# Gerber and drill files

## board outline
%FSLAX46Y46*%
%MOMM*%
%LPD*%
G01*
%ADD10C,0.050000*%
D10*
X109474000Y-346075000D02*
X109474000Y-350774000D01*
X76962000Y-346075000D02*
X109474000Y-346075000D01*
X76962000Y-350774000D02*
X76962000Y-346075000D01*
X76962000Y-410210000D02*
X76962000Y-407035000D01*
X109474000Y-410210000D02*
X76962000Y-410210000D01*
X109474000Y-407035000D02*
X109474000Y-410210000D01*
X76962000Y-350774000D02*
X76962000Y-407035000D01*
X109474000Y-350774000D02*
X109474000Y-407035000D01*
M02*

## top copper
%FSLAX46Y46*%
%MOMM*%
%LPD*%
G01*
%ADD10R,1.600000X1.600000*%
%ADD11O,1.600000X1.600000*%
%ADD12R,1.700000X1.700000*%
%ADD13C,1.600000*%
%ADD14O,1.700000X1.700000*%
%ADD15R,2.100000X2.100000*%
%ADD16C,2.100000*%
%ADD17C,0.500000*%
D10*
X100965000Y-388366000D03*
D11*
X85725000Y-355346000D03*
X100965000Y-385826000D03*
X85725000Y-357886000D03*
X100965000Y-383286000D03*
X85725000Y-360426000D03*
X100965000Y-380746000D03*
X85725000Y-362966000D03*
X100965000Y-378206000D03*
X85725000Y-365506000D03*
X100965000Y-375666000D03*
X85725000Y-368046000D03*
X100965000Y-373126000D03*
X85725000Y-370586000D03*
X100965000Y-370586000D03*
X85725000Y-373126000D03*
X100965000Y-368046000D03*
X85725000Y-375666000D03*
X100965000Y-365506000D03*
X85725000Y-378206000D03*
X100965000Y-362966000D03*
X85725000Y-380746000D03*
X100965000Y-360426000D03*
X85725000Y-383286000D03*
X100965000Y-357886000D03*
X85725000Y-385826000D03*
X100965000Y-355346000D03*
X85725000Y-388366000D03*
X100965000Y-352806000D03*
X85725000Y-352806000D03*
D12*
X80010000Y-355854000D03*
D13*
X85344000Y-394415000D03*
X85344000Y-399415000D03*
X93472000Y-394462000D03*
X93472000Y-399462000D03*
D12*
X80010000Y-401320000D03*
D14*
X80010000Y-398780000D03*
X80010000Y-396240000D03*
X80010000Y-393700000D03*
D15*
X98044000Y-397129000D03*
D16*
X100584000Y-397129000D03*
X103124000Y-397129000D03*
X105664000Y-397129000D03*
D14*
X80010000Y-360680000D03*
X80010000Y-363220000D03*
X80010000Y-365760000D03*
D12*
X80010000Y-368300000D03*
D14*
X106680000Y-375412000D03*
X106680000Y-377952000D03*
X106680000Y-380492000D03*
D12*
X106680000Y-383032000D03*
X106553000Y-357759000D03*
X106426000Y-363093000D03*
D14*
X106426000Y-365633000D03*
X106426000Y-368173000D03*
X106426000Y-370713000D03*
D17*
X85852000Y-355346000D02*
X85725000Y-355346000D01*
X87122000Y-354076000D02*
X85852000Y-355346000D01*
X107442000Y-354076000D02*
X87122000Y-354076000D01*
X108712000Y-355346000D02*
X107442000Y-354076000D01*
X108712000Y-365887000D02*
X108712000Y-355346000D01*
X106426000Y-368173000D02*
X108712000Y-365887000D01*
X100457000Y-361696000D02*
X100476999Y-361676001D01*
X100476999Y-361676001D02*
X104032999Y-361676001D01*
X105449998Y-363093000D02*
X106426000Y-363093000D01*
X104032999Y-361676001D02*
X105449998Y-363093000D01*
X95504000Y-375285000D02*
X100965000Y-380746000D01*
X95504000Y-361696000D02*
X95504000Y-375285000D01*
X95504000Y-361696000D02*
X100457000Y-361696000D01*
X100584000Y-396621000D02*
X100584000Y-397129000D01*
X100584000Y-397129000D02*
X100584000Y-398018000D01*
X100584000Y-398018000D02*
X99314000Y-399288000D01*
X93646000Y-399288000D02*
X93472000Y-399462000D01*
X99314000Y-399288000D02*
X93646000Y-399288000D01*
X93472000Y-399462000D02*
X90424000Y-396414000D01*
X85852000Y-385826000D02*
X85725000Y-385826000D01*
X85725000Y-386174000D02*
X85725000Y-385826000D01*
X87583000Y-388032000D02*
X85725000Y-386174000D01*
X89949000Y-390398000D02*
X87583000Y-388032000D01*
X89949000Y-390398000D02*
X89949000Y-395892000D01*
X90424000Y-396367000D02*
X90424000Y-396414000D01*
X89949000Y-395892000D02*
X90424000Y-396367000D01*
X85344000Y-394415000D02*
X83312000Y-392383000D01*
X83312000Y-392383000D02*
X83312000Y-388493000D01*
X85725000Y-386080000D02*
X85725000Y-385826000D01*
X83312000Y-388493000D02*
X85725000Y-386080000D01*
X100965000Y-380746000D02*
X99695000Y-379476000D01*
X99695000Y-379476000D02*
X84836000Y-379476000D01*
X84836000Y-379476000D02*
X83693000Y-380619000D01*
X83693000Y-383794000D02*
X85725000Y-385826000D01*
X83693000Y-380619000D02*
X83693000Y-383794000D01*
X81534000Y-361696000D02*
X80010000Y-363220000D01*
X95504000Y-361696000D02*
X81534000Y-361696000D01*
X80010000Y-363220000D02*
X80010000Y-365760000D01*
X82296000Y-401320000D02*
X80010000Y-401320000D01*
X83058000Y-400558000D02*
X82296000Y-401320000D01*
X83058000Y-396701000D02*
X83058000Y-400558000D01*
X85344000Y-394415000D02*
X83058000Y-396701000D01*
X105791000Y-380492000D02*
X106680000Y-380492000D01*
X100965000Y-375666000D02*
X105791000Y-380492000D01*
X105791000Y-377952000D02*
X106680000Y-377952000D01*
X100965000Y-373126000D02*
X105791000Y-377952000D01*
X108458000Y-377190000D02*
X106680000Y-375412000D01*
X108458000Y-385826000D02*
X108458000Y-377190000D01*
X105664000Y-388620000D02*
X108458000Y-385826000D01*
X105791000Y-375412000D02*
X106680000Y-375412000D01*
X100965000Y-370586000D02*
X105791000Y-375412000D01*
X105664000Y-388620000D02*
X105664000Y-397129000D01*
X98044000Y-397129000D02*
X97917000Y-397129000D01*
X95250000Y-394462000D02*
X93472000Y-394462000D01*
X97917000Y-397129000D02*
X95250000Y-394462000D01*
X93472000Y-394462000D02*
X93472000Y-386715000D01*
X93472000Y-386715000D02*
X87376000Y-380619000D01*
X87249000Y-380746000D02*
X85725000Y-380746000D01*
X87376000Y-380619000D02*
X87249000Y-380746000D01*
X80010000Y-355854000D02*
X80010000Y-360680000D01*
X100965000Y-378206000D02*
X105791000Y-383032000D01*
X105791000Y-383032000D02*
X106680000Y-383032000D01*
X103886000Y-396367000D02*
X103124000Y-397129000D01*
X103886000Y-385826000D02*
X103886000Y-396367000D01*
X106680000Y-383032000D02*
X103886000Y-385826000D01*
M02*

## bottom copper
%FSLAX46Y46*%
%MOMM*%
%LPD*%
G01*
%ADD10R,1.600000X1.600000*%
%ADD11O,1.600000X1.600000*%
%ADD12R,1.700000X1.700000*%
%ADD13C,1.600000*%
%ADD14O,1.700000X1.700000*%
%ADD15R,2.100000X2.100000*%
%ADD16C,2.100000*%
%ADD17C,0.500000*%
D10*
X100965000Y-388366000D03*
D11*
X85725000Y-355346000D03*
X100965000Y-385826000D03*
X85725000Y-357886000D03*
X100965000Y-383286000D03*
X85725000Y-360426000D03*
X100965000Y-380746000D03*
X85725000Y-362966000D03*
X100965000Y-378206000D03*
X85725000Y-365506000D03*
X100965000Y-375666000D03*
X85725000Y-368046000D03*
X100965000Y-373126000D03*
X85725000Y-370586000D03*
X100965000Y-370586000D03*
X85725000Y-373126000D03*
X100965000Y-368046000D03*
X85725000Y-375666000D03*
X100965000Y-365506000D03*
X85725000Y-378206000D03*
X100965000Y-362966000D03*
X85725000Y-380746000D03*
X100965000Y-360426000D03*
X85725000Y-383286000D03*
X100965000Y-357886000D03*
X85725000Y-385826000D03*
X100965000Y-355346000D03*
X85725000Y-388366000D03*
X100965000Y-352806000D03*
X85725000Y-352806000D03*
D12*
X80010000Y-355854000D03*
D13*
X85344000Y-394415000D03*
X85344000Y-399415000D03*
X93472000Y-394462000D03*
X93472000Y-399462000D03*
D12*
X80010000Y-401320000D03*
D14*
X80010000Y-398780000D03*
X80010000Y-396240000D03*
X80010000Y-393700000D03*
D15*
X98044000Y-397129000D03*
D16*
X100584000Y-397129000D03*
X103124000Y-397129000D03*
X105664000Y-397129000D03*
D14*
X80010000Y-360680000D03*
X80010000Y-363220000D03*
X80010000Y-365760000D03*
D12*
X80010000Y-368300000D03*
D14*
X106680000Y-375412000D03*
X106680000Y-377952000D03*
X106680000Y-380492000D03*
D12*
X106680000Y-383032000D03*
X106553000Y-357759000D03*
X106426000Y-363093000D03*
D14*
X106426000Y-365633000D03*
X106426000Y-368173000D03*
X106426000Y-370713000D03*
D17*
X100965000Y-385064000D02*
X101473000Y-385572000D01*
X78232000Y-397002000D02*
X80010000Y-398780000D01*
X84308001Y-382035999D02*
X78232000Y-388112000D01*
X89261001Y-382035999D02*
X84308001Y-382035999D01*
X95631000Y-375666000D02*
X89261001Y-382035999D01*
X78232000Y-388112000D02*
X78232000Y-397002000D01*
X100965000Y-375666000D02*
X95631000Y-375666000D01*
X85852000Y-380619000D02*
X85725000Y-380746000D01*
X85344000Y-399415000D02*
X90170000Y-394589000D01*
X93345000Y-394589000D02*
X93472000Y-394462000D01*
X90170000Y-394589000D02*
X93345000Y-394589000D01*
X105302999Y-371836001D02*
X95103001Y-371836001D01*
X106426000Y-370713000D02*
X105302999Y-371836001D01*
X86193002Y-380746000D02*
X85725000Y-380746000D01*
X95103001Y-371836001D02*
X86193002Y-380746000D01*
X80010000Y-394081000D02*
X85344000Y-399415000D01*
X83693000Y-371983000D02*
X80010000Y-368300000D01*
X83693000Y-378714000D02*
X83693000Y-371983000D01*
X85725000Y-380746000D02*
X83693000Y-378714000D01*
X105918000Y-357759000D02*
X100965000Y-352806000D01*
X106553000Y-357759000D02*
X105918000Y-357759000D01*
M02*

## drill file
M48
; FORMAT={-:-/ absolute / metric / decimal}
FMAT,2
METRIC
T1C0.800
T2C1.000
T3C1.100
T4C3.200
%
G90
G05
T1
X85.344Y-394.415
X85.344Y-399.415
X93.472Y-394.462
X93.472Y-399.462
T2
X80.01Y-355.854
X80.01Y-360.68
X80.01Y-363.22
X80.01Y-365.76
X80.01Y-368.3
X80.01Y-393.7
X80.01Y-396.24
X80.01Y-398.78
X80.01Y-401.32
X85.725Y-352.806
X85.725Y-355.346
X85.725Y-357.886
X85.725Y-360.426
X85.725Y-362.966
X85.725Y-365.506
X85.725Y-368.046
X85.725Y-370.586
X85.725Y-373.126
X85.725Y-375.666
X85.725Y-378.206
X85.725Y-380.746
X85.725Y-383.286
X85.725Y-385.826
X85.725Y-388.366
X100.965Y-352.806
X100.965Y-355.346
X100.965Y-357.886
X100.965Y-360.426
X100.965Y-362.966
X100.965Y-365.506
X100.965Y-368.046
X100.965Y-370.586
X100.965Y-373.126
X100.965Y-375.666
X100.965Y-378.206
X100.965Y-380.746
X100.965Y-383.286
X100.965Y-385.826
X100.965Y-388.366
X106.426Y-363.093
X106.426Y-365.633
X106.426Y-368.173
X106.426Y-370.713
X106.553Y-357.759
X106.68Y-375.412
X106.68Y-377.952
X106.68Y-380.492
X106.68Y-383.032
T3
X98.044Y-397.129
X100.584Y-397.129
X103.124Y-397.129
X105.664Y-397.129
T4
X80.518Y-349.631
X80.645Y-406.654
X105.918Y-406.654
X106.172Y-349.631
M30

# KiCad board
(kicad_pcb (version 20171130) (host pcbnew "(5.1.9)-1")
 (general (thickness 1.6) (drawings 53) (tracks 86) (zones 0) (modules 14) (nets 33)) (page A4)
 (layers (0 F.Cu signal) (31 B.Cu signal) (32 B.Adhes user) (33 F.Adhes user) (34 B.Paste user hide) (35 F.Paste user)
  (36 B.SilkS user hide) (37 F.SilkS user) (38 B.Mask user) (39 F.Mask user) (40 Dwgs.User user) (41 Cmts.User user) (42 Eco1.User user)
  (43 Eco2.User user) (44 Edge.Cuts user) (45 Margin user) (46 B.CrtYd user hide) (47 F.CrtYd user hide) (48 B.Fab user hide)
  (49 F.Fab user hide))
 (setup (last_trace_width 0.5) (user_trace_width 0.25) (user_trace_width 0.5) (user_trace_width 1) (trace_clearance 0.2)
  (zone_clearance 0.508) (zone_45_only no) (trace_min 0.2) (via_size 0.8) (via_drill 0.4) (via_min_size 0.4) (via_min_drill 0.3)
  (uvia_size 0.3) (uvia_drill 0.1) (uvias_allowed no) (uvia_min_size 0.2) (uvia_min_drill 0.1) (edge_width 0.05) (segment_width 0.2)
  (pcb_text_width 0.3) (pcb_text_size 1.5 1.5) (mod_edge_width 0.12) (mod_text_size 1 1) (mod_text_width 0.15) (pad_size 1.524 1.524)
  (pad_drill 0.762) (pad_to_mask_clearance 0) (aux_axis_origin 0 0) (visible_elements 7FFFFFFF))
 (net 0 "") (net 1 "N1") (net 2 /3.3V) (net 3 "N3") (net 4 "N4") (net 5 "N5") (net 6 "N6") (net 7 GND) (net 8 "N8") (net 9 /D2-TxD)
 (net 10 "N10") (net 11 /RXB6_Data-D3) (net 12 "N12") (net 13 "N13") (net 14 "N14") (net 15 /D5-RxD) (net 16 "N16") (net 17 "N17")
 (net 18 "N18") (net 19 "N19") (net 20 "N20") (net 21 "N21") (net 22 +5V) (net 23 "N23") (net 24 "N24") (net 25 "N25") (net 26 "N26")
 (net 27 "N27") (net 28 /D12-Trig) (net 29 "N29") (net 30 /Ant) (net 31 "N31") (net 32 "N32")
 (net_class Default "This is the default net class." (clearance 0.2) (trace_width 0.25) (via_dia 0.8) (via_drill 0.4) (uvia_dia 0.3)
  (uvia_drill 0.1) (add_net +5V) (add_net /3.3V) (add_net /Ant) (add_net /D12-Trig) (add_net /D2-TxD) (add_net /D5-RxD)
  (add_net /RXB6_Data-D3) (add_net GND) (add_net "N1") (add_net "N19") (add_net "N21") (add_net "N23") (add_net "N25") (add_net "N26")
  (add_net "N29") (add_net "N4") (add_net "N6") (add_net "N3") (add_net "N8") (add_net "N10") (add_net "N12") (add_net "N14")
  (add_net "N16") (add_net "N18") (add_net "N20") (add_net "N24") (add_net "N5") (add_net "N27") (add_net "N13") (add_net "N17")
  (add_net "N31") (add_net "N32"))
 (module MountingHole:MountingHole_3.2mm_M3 (layer F.Cu) (at 106.172 349.631)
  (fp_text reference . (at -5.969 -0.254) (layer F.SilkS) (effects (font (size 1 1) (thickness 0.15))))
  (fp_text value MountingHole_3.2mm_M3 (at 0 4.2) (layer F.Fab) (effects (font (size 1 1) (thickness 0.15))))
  (pad 1 np_thru_hole circle (at 0 0) (size 3.2 3.2) (drill 3.2) (layers *.Cu *.Mask)))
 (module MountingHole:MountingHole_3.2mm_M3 (layer F.Cu) (at 80.518 349.631)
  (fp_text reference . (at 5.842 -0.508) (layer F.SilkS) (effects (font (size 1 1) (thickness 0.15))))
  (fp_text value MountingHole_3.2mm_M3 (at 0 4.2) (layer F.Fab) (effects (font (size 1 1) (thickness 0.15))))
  (pad 1 np_thru_hole circle (at 0 0) (size 3.2 3.2) (drill 3.2) (layers *.Cu *.Mask)))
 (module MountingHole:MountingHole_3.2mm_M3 (layer F.Cu) (at 105.918 406.654)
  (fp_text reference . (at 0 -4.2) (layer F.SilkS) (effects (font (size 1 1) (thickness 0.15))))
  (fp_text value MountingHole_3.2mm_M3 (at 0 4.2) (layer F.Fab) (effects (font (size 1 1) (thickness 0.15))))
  (pad 1 np_thru_hole circle (at 0 0) (size 3.2 3.2) (drill 3.2) (layers *.Cu *.Mask)))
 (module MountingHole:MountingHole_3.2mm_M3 (layer F.Cu) (at 80.645 406.654)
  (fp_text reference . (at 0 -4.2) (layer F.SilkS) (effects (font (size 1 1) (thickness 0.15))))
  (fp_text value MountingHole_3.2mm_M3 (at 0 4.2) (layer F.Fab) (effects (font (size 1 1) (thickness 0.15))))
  (pad 1 np_thru_hole circle (at 0 0) (size 3.2 3.2) (drill 3.2) (layers *.Cu *.Mask)))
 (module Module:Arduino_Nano (layer F.Cu) (at 100.965 388.366 180)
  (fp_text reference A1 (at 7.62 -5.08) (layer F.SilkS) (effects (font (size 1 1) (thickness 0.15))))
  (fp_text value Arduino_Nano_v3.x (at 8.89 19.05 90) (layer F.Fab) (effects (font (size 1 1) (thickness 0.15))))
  (pad 1 thru_hole rect (at 0 0 180) (size 1.6 1.6) (drill 1) (layers *.Cu *.Mask) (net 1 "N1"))
  (pad 17 thru_hole oval (at 15.24 33.02 180) (size 1.6 1.6) (drill 1) (layers *.Cu *.Mask) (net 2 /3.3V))
  (pad 2 thru_hole oval (at 0 2.54 180) (size 1.6 1.6) (drill 1) (layers *.Cu *.Mask) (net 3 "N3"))
  (pad 18 thru_hole oval (at 15.24 30.48 180) (size 1.6 1.6) (drill 1) (layers *.Cu *.Mask) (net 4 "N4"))
  (pad 3 thru_hole oval (at 0 5.08 180) (size 1.6 1.6) (drill 1) (layers *.Cu *.Mask) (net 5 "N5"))
  (pad 19 thru_hole oval (at 15.24 27.94 180) (size 1.6 1.6) (drill 1) (layers *.Cu *.Mask) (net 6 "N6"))
  (pad 4 thru_hole oval (at 0 7.62 180) (size 1.6 1.6) (drill 1) (layers *.Cu *.Mask) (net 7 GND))
  (pad 20 thru_hole oval (at 15.24 25.4 180) (size 1.6 1.6) (drill 1) (layers *.Cu *.Mask) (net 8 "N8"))
  (pad 5 thru_hole oval (at 0 10.16 180) (size 1.6 1.6) (drill 1) (layers *.Cu *.Mask) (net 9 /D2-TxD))
  (pad 21 thru_hole oval (at 15.24 22.86 180) (size 1.6 1.6) (drill 1) (layers *.Cu *.Mask) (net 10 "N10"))
  (pad 6 thru_hole oval (at 0 12.7 180) (size 1.6 1.6) (drill 1) (layers *.Cu *.Mask) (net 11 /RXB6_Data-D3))
  (pad 22 thru_hole oval (at 15.24 20.32 180) (size 1.6 1.6) (drill 1) (layers *.Cu *.Mask) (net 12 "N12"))
  (pad 7 thru_hole oval (at 0 15.24 180) (size 1.6 1.6) (drill 1) (layers *.Cu *.Mask) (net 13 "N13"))
  (pad 23 thru_hole oval (at 15.24 17.78 180) (size 1.6 1.6) (drill 1) (layers *.Cu *.Mask) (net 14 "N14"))
  (pad 8 thru_hole oval (at 0 17.78 180) (size 1.6 1.6) (drill 1) (layers *.Cu *.Mask) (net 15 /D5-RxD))
  (pad 24 thru_hole oval (at 15.24 15.24 180) (size 1.6 1.6) (drill 1) (layers *.Cu *.Mask) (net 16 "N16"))
  (pad 9 thru_hole oval (at 0 20.32 180) (size 1.6 1.6) (drill 1) (layers *.Cu *.Mask) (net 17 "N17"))
  (pad 25 thru_hole oval (at 15.24 12.7 180) (size 1.6 1.6) (drill 1) (layers *.Cu *.Mask) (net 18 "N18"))
  (pad 10 thru_hole oval (at 0 22.86 180) (size 1.6 1.6) (drill 1) (layers *.Cu *.Mask) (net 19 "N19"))
  (pad 26 thru_hole oval (at 15.24 10.16 180) (size 1.6 1.6) (drill 1) (layers *.Cu *.Mask) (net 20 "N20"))
  (pad 11 thru_hole oval (at 0 25.4 180) (size 1.6 1.6) (drill 1) (layers *.Cu *.Mask) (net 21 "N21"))
  (pad 27 thru_hole oval (at 15.24 7.62 180) (size 1.6 1.6) (drill 1) (layers *.Cu *.Mask) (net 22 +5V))
  (pad 12 thru_hole oval (at 0 27.94 180) (size 1.6 1.6) (drill 1) (layers *.Cu *.Mask) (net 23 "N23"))
  (pad 28 thru_hole oval (at 15.24 5.08 180) (size 1.6 1.6) (drill 1) (layers *.Cu *.Mask) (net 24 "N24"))
  (pad 13 thru_hole oval (at 0 30.48 180) (size 1.6 1.6) (drill 1) (layers *.Cu *.Mask) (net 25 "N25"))
  (pad 29 thru_hole oval (at 15.24 2.54 180) (size 1.6 1.6) (drill 1) (layers *.Cu *.Mask) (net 7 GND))
  (pad 14 thru_hole oval (at 0 33.02 180) (size 1.6 1.6) (drill 1) (layers *.Cu *.Mask) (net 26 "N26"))
  (pad 30 thru_hole oval (at 15.24 0 180) (size 1.6 1.6) (drill 1) (layers *.Cu *.Mask) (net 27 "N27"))
  (pad 15 thru_hole oval (at 0 35.56 180) (size 1.6 1.6) (drill 1) (layers *.Cu *.Mask) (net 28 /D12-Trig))
  (pad 16 thru_hole oval (at 15.24 35.56 180) (size 1.6 1.6) (drill 1) (layers *.Cu *.Mask) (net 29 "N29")))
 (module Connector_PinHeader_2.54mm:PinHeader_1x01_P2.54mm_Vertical (layer F.Cu) (at 80.01 355.854)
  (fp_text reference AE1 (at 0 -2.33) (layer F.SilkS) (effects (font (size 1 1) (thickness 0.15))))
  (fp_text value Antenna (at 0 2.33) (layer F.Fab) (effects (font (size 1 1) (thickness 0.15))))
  (pad 1 thru_hole rect (at 0 0) (size 1.7 1.7) (drill 1) (layers *.Cu *.Mask) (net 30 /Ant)))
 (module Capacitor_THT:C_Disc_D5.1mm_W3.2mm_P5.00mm (layer F.Cu) (at 85.344 399.415 90)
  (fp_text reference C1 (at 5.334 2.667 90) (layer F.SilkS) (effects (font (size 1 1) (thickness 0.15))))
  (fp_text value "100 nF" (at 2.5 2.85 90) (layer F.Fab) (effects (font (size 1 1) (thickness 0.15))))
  (pad 2 thru_hole circle (at 5 0 90) (size 1.6 1.6) (drill 0.8) (layers *.Cu *.Mask) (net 7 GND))
  (pad 1 thru_hole circle (at 0 0 90) (size 1.6 1.6) (drill 0.8) (layers *.Cu *.Mask) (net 22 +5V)))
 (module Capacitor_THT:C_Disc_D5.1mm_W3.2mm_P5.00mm (layer F.Cu) (at 93.472 394.462 270)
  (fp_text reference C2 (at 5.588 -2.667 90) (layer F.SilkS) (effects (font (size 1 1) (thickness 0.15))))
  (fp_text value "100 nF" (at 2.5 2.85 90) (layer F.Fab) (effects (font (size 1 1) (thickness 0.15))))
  (pad 1 thru_hole circle (at 0 0 270) (size 1.6 1.6) (drill 0.8) (layers *.Cu *.Mask) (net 22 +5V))
  (pad 2 thru_hole circle (at 5 0 270) (size 1.6 1.6) (drill 0.8) (layers *.Cu *.Mask) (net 7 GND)))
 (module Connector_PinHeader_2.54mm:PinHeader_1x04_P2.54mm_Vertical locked (layer F.Cu) (at 80.01 401.32 180)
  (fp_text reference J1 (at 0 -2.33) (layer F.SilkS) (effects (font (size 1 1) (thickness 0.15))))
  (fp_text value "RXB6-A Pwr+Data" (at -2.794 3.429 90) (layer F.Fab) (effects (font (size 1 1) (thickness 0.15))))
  (pad 1 thru_hole rect (at 0 0 180) (size 1.7 1.7) (drill 1) (layers *.Cu *.Mask) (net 7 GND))
  (pad 2 thru_hole oval (at 0 2.54 180) (size 1.7 1.7) (drill 1) (layers *.Cu *.Mask) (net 11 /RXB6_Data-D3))
  (pad 3 thru_hole oval (at 0 5.08 180) (size 1.7 1.7) (drill 1) (layers *.Cu *.Mask) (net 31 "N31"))
  (pad 4 thru_hole oval (at 0 7.62 180) (size 1.7 1.7) (drill 1) (layers *.Cu *.Mask) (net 22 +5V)))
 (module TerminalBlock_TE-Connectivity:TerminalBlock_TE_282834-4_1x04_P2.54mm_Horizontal (layer F.Cu) (at 98.044 397.129)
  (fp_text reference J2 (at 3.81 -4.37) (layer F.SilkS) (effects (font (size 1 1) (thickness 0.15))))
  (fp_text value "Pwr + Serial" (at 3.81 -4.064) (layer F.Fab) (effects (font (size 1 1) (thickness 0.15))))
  (pad 1 thru_hole rect (at 0 0) (size 2.1 2.1) (drill 1.1) (layers *.Cu *.Mask) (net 22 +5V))
  (pad 2 thru_hole circle (at 2.54 0) (size 2.1 2.1) (drill 1.1) (layers *.Cu *.Mask) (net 7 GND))
  (pad 3 thru_hole circle (at 5.08 0) (size 2.1 2.1) (drill 1.1) (layers *.Cu *.Mask) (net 9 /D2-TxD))
  (pad 4 thru_hole circle (at 7.62 0) (size 2.1 2.1) (drill 1.1) (layers *.Cu *.Mask) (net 15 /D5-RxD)))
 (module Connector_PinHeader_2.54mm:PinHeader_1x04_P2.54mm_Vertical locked (layer F.Cu) (at 80.01 368.3 180)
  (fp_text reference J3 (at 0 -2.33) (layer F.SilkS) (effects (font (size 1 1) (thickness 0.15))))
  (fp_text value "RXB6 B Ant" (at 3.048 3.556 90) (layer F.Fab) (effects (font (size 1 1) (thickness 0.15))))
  (pad 4 thru_hole oval (at 0 7.62 180) (size 1.7 1.7) (drill 1) (layers *.Cu *.Mask) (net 30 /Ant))
  (pad 3 thru_hole oval (at 0 5.08 180) (size 1.7 1.7) (drill 1) (layers *.Cu *.Mask) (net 7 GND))
  (pad 2 thru_hole oval (at 0 2.54 180) (size 1.7 1.7) (drill 1) (layers *.Cu *.Mask) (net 7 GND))
  (pad 1 thru_hole rect (at 0 0 180) (size 1.7 1.7) (drill 1) (layers *.Cu *.Mask) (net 22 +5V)))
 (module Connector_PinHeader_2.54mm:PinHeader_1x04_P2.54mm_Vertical (layer F.Cu) (at 106.68 383.032 180)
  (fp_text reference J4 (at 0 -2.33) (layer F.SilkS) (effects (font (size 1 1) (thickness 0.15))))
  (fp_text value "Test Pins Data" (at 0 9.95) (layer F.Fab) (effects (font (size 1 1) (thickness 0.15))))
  (pad 4 thru_hole oval (at 0 7.62 180) (size 1.7 1.7) (drill 1) (layers *.Cu *.Mask) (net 15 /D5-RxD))
  (pad 3 thru_hole oval (at 0 5.08 180) (size 1.7 1.7) (drill 1) (layers *.Cu *.Mask) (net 13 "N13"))
  (pad 2 thru_hole oval (at 0 2.54 180) (size 1.7 1.7) (drill 1) (layers *.Cu *.Mask) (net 11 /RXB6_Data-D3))
  (pad 1 thru_hole rect (at 0 0 180) (size 1.7 1.7) (drill 1) (layers *.Cu *.Mask) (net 9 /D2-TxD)))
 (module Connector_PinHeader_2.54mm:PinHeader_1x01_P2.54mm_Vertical (layer F.Cu) (at 106.553 357.759)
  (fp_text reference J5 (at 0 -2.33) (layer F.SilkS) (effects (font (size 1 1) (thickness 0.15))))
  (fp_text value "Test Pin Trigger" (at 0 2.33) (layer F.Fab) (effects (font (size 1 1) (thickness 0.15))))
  (pad 1 thru_hole rect (at 0 0) (size 1.7 1.7) (drill 1) (layers *.Cu *.Mask) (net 28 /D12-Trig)))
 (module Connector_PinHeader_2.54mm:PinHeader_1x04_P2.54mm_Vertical (layer F.Cu) (at 106.426 363.093)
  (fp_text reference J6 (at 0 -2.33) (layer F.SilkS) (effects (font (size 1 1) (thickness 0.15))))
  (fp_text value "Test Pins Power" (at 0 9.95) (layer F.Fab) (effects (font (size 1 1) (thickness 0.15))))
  (pad 1 thru_hole rect (at 0 0) (size 1.7 1.7) (drill 1) (layers *.Cu *.Mask) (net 7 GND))
  (pad 2 thru_hole oval (at 0 2.54) (size 1.7 1.7) (drill 1) (layers *.Cu *.Mask) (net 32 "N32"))
  (pad 3 thru_hole oval (at 0 5.08) (size 1.7 1.7) (drill 1) (layers *.Cu *.Mask) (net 2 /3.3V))
  (pad 4 thru_hole oval (at 0 7.62) (size 1.7 1.7) (drill 1) (layers *.Cu *.Mask) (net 22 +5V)))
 (gr_line (start 109.474 346.075) (end 109.474 350.774) (layer Edge.Cuts) (width 0.05))
 (gr_line (start 76.962 346.075) (end 109.474 346.075) (layer Edge.Cuts) (width 0.05))
 (gr_line (start 76.962 350.774) (end 76.962 346.075) (layer Edge.Cuts) (width 0.05))
 (gr_line (start 76.962 410.21) (end 76.962 407.035) (layer Edge.Cuts) (width 0.05))
 (gr_line (start 109.474 410.21) (end 76.962 410.21) (layer Edge.Cuts) (width 0.05))
 (gr_line (start 109.474 407.035) (end 109.474 410.21) (layer Edge.Cuts) (width 0.05))
 (gr_line (start 76.962 350.774) (end 76.962 407.035) (layer Edge.Cuts) (width 0.05))
 (gr_line (start 109.474 350.774) (end 109.474 407.035) (layer Edge.Cuts) (width 0.05))
 (segment (start 85.852 355.346) (end 85.725 355.346) (width 0.5) (layer F.Cu) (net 2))
 (segment (start 87.122 354.076) (end 85.852 355.346) (width 0.5) (layer F.Cu) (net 2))
 (segment (start 107.442 354.076) (end 87.122 354.076) (width 0.5) (layer F.Cu) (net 2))
 (segment (start 108.712 355.346) (end 107.442 354.076) (width 0.5) (layer F.Cu) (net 2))
 (segment (start 108.712 365.887) (end 108.712 355.346) (width 0.5) (layer F.Cu) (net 2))
 (segment (start 106.426 368.173) (end 108.712 365.887) (width 0.5) (layer F.Cu) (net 2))
 (segment (start 100.965 385.064) (end 101.473 385.572) (width 0.5) (layer B.Cu) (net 3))
 (segment (start 100.457 361.696) (end 100.476999 361.676001) (width 0.5) (layer F.Cu) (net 7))
 (segment (start 100.476999 361.676001) (end 104.032999 361.676001) (width 0.5) (layer F.Cu) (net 7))
 (segment (start 105.449998 363.093) (end 106.426 363.093) (width 0.5) (layer F.Cu) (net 7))
 (segment (start 104.032999 361.676001) (end 105.449998 363.093) (width 0.5) (layer F.Cu) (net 7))
 (segment (start 95.504 375.285) (end 100.965 380.746) (width 0.5) (layer F.Cu) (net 7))
 (segment (start 95.504 361.696) (end 95.504 375.285) (width 0.5) (layer F.Cu) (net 7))
 (segment (start 95.504 361.696) (end 100.457 361.696) (width 0.5) (layer F.Cu) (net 7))
 (segment (start 100.584 396.621) (end 100.584 397.129) (width 0.5) (layer F.Cu) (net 7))
 (segment (start 100.584 397.129) (end 100.584 398.018) (width 0.5) (layer F.Cu) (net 7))
 (segment (start 100.584 398.018) (end 99.314 399.288) (width 0.5) (layer F.Cu) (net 7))
 (segment (start 93.646 399.288) (end 93.472 399.462) (width 0.5) (layer F.Cu) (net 7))
 (segment (start 99.314 399.288) (end 93.646 399.288) (width 0.5) (layer F.Cu) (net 7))
 (segment (start 93.472 399.462) (end 90.424 396.414) (width 0.5) (layer F.Cu) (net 7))
 (segment (start 85.852 385.826) (end 85.725 385.826) (width 0.5) (layer F.Cu) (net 7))
 (segment (start 85.725 386.174) (end 85.725 385.826) (width 0.5) (layer F.Cu) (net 7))
 (segment (start 87.583 388.032) (end 85.725 386.174) (width 0.5) (layer F.Cu) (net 7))
 (segment (start 89.949 390.398) (end 87.583 388.032) (width 0.5) (layer F.Cu) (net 7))
 (segment (start 89.949 390.398) (end 89.949 395.892) (width 0.5) (layer F.Cu) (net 7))
 (segment (start 90.424 396.367) (end 90.424 396.414) (width 0.5) (layer F.Cu) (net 7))
 (segment (start 89.949 395.892) (end 90.424 396.367) (width 0.5) (layer F.Cu) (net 7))
 (segment (start 85.344 394.415) (end 83.312 392.383) (width 0.5) (layer F.Cu) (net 7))
 (segment (start 83.312 392.383) (end 83.312 388.493) (width 0.5) (layer F.Cu) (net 7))
 (segment (start 85.725 386.08) (end 85.725 385.826) (width 0.5) (layer F.Cu) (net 7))
 (segment (start 83.312 388.493) (end 85.725 386.08) (width 0.5) (layer F.Cu) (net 7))
 (segment (start 100.965 380.746) (end 99.695 379.476) (width 0.5) (layer F.Cu) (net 7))
 (segment (start 99.695 379.476) (end 84.836 379.476) (width 0.5) (layer F.Cu) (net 7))
 (segment (start 84.836 379.476) (end 83.693 380.619) (width 0.5) (layer F.Cu) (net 7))
 (segment (start 83.693 383.794) (end 85.725 385.826) (width 0.5) (layer F.Cu) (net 7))
 (segment (start 83.693 380.619) (end 83.693 383.794) (width 0.5) (layer F.Cu) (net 7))
 (segment (start 81.534 361.696) (end 80.01 363.22) (width 0.5) (layer F.Cu) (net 7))
 (segment (start 95.504 361.696) (end 81.534 361.696) (width 0.5) (layer F.Cu) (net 7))
 (segment (start 80.01 363.22) (end 80.01 365.76) (width 0.5) (layer F.Cu) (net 7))
 (segment (start 82.296 401.32) (end 80.01 401.32) (width 0.5) (layer F.Cu) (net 7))
 (segment (start 83.058 400.558) (end 82.296 401.32) (width 0.5) (layer F.Cu) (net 7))
 (segment (start 83.058 396.701) (end 83.058 400.558) (width 0.5) (layer F.Cu) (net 7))
 (segment (start 85.344 394.415) (end 83.058 396.701) (width 0.5) (layer F.Cu) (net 7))
 (segment (start 105.791 380.492) (end 106.68 380.492) (width 0.5) (layer F.Cu) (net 11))
 (segment (start 100.965 375.666) (end 105.791 380.492) (width 0.5) (layer F.Cu) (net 11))
 (segment (start 78.232 397.002) (end 80.01 398.78) (width 0.5) (layer B.Cu) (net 11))
 (segment (start 84.308001 382.035999) (end 78.232 388.112) (width 0.5) (layer B.Cu) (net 11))
 (segment (start 89.261001 382.035999) (end 84.308001 382.035999) (width 0.5) (layer B.Cu) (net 11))
 (segment (start 95.631 375.666) (end 89.261001 382.035999) (width 0.5) (layer B.Cu) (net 11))
 (segment (start 78.232 388.112) (end 78.232 397.002) (width 0.5) (layer B.Cu) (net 11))
 (segment (start 100.965 375.666) (end 95.631 375.666) (width 0.5) (layer B.Cu) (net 11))
 (segment (start 105.791 377.952) (end 106.68 377.952) (width 0.5) (layer F.Cu) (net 13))
 (segment (start 100.965 373.126) (end 105.791 377.952) (width 0.5) (layer F.Cu) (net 13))
 (segment (start 108.458 377.19) (end 106.68 375.412) (width 0.5) (layer F.Cu) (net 15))
 (segment (start 108.458 385.826) (end 108.458 377.19) (width 0.5) (layer F.Cu) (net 15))
 (segment (start 105.664 388.62) (end 108.458 385.826) (width 0.5) (layer F.Cu) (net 15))
 (segment (start 105.791 375.412) (end 106.68 375.412) (width 0.5) (layer F.Cu) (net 15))
 (segment (start 100.965 370.586) (end 105.791 375.412) (width 0.5) (layer F.Cu) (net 15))
 (segment (start 105.664 388.62) (end 105.664 397.129) (width 0.5) (layer F.Cu) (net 15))
 (segment (start 85.852 380.619) (end 85.725 380.746) (width 0.5) (layer B.Cu) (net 22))
 (segment (start 98.044 397.129) (end 97.917 397.129) (width 0.5) (layer F.Cu) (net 22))
 (segment (start 95.25 394.462) (end 93.472 394.462) (width 0.5) (layer F.Cu) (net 22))
 (segment (start 97.917 397.129) (end 95.25 394.462) (width 0.5) (layer F.Cu) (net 22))
 (segment (start 93.472 394.462) (end 93.472 386.715) (width 0.5) (layer F.Cu) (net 22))
 (segment (start 93.472 386.715) (end 87.376 380.619) (width 0.5) (layer F.Cu) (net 22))
 (segment (start 87.249 380.746) (end 85.725 380.746) (width 0.5) (layer F.Cu) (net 22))
 (segment (start 87.376 380.619) (end 87.249 380.746) (width 0.5) (layer F.Cu) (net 22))
 (segment (start 85.344 399.415) (end 90.17 394.589) (width 0.5) (layer B.Cu) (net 22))
 (segment (start 93.345 394.589) (end 93.472 394.462) (width 0.5) (layer B.Cu) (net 22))
 (segment (start 90.17 394.589) (end 93.345 394.589) (width 0.5) (layer B.Cu) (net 22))
 (segment (start 105.302999 371.836001) (end 95.103001 371.836001) (width 0.5) (layer B.Cu) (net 22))
 (segment (start 106.426 370.713) (end 105.302999 371.836001) (width 0.5) (layer B.Cu) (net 22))
 (segment (start 86.193002 380.746) (end 85.725 380.746) (width 0.5) (layer B.Cu) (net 22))
 (segment (start 95.103001 371.836001) (end 86.193002 380.746) (width 0.5) (layer B.Cu) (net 22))
 (segment (start 80.01 394.081) (end 85.344 399.415) (width 0.5) (layer B.Cu) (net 22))
 (segment (start 83.693 371.983) (end 80.01 368.3) (width 0.5) (layer B.Cu) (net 22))
 (segment (start 83.693 378.714) (end 83.693 371.983) (width 0.5) (layer B.Cu) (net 22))
 (segment (start 85.725 380.746) (end 83.693 378.714) (width 0.5) (layer B.Cu) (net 22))
 (segment (start 105.918 357.759) (end 100.965 352.806) (width 0.5) (layer B.Cu) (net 28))
 (segment (start 106.553 357.759) (end 105.918 357.759) (width 0.5) (layer B.Cu) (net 28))
 (segment (start 80.01 355.854) (end 80.01 360.68) (width 0.5) (layer F.Cu) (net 30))
 (segment (start 100.965 378.206) (end 105.791 383.032) (width 0.5) (layer F.Cu) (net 9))
 (segment (start 105.791 383.032) (end 106.68 383.032) (width 0.5) (layer F.Cu) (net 9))
 (segment (start 103.886 396.367) (end 103.124 397.129) (width 0.5) (layer F.Cu) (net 9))
 (segment (start 103.886 385.826) (end 103.886 396.367) (width 0.5) (layer F.Cu) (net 9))
 (segment (start 106.68 383.032) (end 103.886 385.826) (width 0.5) (layer F.Cu) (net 9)))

